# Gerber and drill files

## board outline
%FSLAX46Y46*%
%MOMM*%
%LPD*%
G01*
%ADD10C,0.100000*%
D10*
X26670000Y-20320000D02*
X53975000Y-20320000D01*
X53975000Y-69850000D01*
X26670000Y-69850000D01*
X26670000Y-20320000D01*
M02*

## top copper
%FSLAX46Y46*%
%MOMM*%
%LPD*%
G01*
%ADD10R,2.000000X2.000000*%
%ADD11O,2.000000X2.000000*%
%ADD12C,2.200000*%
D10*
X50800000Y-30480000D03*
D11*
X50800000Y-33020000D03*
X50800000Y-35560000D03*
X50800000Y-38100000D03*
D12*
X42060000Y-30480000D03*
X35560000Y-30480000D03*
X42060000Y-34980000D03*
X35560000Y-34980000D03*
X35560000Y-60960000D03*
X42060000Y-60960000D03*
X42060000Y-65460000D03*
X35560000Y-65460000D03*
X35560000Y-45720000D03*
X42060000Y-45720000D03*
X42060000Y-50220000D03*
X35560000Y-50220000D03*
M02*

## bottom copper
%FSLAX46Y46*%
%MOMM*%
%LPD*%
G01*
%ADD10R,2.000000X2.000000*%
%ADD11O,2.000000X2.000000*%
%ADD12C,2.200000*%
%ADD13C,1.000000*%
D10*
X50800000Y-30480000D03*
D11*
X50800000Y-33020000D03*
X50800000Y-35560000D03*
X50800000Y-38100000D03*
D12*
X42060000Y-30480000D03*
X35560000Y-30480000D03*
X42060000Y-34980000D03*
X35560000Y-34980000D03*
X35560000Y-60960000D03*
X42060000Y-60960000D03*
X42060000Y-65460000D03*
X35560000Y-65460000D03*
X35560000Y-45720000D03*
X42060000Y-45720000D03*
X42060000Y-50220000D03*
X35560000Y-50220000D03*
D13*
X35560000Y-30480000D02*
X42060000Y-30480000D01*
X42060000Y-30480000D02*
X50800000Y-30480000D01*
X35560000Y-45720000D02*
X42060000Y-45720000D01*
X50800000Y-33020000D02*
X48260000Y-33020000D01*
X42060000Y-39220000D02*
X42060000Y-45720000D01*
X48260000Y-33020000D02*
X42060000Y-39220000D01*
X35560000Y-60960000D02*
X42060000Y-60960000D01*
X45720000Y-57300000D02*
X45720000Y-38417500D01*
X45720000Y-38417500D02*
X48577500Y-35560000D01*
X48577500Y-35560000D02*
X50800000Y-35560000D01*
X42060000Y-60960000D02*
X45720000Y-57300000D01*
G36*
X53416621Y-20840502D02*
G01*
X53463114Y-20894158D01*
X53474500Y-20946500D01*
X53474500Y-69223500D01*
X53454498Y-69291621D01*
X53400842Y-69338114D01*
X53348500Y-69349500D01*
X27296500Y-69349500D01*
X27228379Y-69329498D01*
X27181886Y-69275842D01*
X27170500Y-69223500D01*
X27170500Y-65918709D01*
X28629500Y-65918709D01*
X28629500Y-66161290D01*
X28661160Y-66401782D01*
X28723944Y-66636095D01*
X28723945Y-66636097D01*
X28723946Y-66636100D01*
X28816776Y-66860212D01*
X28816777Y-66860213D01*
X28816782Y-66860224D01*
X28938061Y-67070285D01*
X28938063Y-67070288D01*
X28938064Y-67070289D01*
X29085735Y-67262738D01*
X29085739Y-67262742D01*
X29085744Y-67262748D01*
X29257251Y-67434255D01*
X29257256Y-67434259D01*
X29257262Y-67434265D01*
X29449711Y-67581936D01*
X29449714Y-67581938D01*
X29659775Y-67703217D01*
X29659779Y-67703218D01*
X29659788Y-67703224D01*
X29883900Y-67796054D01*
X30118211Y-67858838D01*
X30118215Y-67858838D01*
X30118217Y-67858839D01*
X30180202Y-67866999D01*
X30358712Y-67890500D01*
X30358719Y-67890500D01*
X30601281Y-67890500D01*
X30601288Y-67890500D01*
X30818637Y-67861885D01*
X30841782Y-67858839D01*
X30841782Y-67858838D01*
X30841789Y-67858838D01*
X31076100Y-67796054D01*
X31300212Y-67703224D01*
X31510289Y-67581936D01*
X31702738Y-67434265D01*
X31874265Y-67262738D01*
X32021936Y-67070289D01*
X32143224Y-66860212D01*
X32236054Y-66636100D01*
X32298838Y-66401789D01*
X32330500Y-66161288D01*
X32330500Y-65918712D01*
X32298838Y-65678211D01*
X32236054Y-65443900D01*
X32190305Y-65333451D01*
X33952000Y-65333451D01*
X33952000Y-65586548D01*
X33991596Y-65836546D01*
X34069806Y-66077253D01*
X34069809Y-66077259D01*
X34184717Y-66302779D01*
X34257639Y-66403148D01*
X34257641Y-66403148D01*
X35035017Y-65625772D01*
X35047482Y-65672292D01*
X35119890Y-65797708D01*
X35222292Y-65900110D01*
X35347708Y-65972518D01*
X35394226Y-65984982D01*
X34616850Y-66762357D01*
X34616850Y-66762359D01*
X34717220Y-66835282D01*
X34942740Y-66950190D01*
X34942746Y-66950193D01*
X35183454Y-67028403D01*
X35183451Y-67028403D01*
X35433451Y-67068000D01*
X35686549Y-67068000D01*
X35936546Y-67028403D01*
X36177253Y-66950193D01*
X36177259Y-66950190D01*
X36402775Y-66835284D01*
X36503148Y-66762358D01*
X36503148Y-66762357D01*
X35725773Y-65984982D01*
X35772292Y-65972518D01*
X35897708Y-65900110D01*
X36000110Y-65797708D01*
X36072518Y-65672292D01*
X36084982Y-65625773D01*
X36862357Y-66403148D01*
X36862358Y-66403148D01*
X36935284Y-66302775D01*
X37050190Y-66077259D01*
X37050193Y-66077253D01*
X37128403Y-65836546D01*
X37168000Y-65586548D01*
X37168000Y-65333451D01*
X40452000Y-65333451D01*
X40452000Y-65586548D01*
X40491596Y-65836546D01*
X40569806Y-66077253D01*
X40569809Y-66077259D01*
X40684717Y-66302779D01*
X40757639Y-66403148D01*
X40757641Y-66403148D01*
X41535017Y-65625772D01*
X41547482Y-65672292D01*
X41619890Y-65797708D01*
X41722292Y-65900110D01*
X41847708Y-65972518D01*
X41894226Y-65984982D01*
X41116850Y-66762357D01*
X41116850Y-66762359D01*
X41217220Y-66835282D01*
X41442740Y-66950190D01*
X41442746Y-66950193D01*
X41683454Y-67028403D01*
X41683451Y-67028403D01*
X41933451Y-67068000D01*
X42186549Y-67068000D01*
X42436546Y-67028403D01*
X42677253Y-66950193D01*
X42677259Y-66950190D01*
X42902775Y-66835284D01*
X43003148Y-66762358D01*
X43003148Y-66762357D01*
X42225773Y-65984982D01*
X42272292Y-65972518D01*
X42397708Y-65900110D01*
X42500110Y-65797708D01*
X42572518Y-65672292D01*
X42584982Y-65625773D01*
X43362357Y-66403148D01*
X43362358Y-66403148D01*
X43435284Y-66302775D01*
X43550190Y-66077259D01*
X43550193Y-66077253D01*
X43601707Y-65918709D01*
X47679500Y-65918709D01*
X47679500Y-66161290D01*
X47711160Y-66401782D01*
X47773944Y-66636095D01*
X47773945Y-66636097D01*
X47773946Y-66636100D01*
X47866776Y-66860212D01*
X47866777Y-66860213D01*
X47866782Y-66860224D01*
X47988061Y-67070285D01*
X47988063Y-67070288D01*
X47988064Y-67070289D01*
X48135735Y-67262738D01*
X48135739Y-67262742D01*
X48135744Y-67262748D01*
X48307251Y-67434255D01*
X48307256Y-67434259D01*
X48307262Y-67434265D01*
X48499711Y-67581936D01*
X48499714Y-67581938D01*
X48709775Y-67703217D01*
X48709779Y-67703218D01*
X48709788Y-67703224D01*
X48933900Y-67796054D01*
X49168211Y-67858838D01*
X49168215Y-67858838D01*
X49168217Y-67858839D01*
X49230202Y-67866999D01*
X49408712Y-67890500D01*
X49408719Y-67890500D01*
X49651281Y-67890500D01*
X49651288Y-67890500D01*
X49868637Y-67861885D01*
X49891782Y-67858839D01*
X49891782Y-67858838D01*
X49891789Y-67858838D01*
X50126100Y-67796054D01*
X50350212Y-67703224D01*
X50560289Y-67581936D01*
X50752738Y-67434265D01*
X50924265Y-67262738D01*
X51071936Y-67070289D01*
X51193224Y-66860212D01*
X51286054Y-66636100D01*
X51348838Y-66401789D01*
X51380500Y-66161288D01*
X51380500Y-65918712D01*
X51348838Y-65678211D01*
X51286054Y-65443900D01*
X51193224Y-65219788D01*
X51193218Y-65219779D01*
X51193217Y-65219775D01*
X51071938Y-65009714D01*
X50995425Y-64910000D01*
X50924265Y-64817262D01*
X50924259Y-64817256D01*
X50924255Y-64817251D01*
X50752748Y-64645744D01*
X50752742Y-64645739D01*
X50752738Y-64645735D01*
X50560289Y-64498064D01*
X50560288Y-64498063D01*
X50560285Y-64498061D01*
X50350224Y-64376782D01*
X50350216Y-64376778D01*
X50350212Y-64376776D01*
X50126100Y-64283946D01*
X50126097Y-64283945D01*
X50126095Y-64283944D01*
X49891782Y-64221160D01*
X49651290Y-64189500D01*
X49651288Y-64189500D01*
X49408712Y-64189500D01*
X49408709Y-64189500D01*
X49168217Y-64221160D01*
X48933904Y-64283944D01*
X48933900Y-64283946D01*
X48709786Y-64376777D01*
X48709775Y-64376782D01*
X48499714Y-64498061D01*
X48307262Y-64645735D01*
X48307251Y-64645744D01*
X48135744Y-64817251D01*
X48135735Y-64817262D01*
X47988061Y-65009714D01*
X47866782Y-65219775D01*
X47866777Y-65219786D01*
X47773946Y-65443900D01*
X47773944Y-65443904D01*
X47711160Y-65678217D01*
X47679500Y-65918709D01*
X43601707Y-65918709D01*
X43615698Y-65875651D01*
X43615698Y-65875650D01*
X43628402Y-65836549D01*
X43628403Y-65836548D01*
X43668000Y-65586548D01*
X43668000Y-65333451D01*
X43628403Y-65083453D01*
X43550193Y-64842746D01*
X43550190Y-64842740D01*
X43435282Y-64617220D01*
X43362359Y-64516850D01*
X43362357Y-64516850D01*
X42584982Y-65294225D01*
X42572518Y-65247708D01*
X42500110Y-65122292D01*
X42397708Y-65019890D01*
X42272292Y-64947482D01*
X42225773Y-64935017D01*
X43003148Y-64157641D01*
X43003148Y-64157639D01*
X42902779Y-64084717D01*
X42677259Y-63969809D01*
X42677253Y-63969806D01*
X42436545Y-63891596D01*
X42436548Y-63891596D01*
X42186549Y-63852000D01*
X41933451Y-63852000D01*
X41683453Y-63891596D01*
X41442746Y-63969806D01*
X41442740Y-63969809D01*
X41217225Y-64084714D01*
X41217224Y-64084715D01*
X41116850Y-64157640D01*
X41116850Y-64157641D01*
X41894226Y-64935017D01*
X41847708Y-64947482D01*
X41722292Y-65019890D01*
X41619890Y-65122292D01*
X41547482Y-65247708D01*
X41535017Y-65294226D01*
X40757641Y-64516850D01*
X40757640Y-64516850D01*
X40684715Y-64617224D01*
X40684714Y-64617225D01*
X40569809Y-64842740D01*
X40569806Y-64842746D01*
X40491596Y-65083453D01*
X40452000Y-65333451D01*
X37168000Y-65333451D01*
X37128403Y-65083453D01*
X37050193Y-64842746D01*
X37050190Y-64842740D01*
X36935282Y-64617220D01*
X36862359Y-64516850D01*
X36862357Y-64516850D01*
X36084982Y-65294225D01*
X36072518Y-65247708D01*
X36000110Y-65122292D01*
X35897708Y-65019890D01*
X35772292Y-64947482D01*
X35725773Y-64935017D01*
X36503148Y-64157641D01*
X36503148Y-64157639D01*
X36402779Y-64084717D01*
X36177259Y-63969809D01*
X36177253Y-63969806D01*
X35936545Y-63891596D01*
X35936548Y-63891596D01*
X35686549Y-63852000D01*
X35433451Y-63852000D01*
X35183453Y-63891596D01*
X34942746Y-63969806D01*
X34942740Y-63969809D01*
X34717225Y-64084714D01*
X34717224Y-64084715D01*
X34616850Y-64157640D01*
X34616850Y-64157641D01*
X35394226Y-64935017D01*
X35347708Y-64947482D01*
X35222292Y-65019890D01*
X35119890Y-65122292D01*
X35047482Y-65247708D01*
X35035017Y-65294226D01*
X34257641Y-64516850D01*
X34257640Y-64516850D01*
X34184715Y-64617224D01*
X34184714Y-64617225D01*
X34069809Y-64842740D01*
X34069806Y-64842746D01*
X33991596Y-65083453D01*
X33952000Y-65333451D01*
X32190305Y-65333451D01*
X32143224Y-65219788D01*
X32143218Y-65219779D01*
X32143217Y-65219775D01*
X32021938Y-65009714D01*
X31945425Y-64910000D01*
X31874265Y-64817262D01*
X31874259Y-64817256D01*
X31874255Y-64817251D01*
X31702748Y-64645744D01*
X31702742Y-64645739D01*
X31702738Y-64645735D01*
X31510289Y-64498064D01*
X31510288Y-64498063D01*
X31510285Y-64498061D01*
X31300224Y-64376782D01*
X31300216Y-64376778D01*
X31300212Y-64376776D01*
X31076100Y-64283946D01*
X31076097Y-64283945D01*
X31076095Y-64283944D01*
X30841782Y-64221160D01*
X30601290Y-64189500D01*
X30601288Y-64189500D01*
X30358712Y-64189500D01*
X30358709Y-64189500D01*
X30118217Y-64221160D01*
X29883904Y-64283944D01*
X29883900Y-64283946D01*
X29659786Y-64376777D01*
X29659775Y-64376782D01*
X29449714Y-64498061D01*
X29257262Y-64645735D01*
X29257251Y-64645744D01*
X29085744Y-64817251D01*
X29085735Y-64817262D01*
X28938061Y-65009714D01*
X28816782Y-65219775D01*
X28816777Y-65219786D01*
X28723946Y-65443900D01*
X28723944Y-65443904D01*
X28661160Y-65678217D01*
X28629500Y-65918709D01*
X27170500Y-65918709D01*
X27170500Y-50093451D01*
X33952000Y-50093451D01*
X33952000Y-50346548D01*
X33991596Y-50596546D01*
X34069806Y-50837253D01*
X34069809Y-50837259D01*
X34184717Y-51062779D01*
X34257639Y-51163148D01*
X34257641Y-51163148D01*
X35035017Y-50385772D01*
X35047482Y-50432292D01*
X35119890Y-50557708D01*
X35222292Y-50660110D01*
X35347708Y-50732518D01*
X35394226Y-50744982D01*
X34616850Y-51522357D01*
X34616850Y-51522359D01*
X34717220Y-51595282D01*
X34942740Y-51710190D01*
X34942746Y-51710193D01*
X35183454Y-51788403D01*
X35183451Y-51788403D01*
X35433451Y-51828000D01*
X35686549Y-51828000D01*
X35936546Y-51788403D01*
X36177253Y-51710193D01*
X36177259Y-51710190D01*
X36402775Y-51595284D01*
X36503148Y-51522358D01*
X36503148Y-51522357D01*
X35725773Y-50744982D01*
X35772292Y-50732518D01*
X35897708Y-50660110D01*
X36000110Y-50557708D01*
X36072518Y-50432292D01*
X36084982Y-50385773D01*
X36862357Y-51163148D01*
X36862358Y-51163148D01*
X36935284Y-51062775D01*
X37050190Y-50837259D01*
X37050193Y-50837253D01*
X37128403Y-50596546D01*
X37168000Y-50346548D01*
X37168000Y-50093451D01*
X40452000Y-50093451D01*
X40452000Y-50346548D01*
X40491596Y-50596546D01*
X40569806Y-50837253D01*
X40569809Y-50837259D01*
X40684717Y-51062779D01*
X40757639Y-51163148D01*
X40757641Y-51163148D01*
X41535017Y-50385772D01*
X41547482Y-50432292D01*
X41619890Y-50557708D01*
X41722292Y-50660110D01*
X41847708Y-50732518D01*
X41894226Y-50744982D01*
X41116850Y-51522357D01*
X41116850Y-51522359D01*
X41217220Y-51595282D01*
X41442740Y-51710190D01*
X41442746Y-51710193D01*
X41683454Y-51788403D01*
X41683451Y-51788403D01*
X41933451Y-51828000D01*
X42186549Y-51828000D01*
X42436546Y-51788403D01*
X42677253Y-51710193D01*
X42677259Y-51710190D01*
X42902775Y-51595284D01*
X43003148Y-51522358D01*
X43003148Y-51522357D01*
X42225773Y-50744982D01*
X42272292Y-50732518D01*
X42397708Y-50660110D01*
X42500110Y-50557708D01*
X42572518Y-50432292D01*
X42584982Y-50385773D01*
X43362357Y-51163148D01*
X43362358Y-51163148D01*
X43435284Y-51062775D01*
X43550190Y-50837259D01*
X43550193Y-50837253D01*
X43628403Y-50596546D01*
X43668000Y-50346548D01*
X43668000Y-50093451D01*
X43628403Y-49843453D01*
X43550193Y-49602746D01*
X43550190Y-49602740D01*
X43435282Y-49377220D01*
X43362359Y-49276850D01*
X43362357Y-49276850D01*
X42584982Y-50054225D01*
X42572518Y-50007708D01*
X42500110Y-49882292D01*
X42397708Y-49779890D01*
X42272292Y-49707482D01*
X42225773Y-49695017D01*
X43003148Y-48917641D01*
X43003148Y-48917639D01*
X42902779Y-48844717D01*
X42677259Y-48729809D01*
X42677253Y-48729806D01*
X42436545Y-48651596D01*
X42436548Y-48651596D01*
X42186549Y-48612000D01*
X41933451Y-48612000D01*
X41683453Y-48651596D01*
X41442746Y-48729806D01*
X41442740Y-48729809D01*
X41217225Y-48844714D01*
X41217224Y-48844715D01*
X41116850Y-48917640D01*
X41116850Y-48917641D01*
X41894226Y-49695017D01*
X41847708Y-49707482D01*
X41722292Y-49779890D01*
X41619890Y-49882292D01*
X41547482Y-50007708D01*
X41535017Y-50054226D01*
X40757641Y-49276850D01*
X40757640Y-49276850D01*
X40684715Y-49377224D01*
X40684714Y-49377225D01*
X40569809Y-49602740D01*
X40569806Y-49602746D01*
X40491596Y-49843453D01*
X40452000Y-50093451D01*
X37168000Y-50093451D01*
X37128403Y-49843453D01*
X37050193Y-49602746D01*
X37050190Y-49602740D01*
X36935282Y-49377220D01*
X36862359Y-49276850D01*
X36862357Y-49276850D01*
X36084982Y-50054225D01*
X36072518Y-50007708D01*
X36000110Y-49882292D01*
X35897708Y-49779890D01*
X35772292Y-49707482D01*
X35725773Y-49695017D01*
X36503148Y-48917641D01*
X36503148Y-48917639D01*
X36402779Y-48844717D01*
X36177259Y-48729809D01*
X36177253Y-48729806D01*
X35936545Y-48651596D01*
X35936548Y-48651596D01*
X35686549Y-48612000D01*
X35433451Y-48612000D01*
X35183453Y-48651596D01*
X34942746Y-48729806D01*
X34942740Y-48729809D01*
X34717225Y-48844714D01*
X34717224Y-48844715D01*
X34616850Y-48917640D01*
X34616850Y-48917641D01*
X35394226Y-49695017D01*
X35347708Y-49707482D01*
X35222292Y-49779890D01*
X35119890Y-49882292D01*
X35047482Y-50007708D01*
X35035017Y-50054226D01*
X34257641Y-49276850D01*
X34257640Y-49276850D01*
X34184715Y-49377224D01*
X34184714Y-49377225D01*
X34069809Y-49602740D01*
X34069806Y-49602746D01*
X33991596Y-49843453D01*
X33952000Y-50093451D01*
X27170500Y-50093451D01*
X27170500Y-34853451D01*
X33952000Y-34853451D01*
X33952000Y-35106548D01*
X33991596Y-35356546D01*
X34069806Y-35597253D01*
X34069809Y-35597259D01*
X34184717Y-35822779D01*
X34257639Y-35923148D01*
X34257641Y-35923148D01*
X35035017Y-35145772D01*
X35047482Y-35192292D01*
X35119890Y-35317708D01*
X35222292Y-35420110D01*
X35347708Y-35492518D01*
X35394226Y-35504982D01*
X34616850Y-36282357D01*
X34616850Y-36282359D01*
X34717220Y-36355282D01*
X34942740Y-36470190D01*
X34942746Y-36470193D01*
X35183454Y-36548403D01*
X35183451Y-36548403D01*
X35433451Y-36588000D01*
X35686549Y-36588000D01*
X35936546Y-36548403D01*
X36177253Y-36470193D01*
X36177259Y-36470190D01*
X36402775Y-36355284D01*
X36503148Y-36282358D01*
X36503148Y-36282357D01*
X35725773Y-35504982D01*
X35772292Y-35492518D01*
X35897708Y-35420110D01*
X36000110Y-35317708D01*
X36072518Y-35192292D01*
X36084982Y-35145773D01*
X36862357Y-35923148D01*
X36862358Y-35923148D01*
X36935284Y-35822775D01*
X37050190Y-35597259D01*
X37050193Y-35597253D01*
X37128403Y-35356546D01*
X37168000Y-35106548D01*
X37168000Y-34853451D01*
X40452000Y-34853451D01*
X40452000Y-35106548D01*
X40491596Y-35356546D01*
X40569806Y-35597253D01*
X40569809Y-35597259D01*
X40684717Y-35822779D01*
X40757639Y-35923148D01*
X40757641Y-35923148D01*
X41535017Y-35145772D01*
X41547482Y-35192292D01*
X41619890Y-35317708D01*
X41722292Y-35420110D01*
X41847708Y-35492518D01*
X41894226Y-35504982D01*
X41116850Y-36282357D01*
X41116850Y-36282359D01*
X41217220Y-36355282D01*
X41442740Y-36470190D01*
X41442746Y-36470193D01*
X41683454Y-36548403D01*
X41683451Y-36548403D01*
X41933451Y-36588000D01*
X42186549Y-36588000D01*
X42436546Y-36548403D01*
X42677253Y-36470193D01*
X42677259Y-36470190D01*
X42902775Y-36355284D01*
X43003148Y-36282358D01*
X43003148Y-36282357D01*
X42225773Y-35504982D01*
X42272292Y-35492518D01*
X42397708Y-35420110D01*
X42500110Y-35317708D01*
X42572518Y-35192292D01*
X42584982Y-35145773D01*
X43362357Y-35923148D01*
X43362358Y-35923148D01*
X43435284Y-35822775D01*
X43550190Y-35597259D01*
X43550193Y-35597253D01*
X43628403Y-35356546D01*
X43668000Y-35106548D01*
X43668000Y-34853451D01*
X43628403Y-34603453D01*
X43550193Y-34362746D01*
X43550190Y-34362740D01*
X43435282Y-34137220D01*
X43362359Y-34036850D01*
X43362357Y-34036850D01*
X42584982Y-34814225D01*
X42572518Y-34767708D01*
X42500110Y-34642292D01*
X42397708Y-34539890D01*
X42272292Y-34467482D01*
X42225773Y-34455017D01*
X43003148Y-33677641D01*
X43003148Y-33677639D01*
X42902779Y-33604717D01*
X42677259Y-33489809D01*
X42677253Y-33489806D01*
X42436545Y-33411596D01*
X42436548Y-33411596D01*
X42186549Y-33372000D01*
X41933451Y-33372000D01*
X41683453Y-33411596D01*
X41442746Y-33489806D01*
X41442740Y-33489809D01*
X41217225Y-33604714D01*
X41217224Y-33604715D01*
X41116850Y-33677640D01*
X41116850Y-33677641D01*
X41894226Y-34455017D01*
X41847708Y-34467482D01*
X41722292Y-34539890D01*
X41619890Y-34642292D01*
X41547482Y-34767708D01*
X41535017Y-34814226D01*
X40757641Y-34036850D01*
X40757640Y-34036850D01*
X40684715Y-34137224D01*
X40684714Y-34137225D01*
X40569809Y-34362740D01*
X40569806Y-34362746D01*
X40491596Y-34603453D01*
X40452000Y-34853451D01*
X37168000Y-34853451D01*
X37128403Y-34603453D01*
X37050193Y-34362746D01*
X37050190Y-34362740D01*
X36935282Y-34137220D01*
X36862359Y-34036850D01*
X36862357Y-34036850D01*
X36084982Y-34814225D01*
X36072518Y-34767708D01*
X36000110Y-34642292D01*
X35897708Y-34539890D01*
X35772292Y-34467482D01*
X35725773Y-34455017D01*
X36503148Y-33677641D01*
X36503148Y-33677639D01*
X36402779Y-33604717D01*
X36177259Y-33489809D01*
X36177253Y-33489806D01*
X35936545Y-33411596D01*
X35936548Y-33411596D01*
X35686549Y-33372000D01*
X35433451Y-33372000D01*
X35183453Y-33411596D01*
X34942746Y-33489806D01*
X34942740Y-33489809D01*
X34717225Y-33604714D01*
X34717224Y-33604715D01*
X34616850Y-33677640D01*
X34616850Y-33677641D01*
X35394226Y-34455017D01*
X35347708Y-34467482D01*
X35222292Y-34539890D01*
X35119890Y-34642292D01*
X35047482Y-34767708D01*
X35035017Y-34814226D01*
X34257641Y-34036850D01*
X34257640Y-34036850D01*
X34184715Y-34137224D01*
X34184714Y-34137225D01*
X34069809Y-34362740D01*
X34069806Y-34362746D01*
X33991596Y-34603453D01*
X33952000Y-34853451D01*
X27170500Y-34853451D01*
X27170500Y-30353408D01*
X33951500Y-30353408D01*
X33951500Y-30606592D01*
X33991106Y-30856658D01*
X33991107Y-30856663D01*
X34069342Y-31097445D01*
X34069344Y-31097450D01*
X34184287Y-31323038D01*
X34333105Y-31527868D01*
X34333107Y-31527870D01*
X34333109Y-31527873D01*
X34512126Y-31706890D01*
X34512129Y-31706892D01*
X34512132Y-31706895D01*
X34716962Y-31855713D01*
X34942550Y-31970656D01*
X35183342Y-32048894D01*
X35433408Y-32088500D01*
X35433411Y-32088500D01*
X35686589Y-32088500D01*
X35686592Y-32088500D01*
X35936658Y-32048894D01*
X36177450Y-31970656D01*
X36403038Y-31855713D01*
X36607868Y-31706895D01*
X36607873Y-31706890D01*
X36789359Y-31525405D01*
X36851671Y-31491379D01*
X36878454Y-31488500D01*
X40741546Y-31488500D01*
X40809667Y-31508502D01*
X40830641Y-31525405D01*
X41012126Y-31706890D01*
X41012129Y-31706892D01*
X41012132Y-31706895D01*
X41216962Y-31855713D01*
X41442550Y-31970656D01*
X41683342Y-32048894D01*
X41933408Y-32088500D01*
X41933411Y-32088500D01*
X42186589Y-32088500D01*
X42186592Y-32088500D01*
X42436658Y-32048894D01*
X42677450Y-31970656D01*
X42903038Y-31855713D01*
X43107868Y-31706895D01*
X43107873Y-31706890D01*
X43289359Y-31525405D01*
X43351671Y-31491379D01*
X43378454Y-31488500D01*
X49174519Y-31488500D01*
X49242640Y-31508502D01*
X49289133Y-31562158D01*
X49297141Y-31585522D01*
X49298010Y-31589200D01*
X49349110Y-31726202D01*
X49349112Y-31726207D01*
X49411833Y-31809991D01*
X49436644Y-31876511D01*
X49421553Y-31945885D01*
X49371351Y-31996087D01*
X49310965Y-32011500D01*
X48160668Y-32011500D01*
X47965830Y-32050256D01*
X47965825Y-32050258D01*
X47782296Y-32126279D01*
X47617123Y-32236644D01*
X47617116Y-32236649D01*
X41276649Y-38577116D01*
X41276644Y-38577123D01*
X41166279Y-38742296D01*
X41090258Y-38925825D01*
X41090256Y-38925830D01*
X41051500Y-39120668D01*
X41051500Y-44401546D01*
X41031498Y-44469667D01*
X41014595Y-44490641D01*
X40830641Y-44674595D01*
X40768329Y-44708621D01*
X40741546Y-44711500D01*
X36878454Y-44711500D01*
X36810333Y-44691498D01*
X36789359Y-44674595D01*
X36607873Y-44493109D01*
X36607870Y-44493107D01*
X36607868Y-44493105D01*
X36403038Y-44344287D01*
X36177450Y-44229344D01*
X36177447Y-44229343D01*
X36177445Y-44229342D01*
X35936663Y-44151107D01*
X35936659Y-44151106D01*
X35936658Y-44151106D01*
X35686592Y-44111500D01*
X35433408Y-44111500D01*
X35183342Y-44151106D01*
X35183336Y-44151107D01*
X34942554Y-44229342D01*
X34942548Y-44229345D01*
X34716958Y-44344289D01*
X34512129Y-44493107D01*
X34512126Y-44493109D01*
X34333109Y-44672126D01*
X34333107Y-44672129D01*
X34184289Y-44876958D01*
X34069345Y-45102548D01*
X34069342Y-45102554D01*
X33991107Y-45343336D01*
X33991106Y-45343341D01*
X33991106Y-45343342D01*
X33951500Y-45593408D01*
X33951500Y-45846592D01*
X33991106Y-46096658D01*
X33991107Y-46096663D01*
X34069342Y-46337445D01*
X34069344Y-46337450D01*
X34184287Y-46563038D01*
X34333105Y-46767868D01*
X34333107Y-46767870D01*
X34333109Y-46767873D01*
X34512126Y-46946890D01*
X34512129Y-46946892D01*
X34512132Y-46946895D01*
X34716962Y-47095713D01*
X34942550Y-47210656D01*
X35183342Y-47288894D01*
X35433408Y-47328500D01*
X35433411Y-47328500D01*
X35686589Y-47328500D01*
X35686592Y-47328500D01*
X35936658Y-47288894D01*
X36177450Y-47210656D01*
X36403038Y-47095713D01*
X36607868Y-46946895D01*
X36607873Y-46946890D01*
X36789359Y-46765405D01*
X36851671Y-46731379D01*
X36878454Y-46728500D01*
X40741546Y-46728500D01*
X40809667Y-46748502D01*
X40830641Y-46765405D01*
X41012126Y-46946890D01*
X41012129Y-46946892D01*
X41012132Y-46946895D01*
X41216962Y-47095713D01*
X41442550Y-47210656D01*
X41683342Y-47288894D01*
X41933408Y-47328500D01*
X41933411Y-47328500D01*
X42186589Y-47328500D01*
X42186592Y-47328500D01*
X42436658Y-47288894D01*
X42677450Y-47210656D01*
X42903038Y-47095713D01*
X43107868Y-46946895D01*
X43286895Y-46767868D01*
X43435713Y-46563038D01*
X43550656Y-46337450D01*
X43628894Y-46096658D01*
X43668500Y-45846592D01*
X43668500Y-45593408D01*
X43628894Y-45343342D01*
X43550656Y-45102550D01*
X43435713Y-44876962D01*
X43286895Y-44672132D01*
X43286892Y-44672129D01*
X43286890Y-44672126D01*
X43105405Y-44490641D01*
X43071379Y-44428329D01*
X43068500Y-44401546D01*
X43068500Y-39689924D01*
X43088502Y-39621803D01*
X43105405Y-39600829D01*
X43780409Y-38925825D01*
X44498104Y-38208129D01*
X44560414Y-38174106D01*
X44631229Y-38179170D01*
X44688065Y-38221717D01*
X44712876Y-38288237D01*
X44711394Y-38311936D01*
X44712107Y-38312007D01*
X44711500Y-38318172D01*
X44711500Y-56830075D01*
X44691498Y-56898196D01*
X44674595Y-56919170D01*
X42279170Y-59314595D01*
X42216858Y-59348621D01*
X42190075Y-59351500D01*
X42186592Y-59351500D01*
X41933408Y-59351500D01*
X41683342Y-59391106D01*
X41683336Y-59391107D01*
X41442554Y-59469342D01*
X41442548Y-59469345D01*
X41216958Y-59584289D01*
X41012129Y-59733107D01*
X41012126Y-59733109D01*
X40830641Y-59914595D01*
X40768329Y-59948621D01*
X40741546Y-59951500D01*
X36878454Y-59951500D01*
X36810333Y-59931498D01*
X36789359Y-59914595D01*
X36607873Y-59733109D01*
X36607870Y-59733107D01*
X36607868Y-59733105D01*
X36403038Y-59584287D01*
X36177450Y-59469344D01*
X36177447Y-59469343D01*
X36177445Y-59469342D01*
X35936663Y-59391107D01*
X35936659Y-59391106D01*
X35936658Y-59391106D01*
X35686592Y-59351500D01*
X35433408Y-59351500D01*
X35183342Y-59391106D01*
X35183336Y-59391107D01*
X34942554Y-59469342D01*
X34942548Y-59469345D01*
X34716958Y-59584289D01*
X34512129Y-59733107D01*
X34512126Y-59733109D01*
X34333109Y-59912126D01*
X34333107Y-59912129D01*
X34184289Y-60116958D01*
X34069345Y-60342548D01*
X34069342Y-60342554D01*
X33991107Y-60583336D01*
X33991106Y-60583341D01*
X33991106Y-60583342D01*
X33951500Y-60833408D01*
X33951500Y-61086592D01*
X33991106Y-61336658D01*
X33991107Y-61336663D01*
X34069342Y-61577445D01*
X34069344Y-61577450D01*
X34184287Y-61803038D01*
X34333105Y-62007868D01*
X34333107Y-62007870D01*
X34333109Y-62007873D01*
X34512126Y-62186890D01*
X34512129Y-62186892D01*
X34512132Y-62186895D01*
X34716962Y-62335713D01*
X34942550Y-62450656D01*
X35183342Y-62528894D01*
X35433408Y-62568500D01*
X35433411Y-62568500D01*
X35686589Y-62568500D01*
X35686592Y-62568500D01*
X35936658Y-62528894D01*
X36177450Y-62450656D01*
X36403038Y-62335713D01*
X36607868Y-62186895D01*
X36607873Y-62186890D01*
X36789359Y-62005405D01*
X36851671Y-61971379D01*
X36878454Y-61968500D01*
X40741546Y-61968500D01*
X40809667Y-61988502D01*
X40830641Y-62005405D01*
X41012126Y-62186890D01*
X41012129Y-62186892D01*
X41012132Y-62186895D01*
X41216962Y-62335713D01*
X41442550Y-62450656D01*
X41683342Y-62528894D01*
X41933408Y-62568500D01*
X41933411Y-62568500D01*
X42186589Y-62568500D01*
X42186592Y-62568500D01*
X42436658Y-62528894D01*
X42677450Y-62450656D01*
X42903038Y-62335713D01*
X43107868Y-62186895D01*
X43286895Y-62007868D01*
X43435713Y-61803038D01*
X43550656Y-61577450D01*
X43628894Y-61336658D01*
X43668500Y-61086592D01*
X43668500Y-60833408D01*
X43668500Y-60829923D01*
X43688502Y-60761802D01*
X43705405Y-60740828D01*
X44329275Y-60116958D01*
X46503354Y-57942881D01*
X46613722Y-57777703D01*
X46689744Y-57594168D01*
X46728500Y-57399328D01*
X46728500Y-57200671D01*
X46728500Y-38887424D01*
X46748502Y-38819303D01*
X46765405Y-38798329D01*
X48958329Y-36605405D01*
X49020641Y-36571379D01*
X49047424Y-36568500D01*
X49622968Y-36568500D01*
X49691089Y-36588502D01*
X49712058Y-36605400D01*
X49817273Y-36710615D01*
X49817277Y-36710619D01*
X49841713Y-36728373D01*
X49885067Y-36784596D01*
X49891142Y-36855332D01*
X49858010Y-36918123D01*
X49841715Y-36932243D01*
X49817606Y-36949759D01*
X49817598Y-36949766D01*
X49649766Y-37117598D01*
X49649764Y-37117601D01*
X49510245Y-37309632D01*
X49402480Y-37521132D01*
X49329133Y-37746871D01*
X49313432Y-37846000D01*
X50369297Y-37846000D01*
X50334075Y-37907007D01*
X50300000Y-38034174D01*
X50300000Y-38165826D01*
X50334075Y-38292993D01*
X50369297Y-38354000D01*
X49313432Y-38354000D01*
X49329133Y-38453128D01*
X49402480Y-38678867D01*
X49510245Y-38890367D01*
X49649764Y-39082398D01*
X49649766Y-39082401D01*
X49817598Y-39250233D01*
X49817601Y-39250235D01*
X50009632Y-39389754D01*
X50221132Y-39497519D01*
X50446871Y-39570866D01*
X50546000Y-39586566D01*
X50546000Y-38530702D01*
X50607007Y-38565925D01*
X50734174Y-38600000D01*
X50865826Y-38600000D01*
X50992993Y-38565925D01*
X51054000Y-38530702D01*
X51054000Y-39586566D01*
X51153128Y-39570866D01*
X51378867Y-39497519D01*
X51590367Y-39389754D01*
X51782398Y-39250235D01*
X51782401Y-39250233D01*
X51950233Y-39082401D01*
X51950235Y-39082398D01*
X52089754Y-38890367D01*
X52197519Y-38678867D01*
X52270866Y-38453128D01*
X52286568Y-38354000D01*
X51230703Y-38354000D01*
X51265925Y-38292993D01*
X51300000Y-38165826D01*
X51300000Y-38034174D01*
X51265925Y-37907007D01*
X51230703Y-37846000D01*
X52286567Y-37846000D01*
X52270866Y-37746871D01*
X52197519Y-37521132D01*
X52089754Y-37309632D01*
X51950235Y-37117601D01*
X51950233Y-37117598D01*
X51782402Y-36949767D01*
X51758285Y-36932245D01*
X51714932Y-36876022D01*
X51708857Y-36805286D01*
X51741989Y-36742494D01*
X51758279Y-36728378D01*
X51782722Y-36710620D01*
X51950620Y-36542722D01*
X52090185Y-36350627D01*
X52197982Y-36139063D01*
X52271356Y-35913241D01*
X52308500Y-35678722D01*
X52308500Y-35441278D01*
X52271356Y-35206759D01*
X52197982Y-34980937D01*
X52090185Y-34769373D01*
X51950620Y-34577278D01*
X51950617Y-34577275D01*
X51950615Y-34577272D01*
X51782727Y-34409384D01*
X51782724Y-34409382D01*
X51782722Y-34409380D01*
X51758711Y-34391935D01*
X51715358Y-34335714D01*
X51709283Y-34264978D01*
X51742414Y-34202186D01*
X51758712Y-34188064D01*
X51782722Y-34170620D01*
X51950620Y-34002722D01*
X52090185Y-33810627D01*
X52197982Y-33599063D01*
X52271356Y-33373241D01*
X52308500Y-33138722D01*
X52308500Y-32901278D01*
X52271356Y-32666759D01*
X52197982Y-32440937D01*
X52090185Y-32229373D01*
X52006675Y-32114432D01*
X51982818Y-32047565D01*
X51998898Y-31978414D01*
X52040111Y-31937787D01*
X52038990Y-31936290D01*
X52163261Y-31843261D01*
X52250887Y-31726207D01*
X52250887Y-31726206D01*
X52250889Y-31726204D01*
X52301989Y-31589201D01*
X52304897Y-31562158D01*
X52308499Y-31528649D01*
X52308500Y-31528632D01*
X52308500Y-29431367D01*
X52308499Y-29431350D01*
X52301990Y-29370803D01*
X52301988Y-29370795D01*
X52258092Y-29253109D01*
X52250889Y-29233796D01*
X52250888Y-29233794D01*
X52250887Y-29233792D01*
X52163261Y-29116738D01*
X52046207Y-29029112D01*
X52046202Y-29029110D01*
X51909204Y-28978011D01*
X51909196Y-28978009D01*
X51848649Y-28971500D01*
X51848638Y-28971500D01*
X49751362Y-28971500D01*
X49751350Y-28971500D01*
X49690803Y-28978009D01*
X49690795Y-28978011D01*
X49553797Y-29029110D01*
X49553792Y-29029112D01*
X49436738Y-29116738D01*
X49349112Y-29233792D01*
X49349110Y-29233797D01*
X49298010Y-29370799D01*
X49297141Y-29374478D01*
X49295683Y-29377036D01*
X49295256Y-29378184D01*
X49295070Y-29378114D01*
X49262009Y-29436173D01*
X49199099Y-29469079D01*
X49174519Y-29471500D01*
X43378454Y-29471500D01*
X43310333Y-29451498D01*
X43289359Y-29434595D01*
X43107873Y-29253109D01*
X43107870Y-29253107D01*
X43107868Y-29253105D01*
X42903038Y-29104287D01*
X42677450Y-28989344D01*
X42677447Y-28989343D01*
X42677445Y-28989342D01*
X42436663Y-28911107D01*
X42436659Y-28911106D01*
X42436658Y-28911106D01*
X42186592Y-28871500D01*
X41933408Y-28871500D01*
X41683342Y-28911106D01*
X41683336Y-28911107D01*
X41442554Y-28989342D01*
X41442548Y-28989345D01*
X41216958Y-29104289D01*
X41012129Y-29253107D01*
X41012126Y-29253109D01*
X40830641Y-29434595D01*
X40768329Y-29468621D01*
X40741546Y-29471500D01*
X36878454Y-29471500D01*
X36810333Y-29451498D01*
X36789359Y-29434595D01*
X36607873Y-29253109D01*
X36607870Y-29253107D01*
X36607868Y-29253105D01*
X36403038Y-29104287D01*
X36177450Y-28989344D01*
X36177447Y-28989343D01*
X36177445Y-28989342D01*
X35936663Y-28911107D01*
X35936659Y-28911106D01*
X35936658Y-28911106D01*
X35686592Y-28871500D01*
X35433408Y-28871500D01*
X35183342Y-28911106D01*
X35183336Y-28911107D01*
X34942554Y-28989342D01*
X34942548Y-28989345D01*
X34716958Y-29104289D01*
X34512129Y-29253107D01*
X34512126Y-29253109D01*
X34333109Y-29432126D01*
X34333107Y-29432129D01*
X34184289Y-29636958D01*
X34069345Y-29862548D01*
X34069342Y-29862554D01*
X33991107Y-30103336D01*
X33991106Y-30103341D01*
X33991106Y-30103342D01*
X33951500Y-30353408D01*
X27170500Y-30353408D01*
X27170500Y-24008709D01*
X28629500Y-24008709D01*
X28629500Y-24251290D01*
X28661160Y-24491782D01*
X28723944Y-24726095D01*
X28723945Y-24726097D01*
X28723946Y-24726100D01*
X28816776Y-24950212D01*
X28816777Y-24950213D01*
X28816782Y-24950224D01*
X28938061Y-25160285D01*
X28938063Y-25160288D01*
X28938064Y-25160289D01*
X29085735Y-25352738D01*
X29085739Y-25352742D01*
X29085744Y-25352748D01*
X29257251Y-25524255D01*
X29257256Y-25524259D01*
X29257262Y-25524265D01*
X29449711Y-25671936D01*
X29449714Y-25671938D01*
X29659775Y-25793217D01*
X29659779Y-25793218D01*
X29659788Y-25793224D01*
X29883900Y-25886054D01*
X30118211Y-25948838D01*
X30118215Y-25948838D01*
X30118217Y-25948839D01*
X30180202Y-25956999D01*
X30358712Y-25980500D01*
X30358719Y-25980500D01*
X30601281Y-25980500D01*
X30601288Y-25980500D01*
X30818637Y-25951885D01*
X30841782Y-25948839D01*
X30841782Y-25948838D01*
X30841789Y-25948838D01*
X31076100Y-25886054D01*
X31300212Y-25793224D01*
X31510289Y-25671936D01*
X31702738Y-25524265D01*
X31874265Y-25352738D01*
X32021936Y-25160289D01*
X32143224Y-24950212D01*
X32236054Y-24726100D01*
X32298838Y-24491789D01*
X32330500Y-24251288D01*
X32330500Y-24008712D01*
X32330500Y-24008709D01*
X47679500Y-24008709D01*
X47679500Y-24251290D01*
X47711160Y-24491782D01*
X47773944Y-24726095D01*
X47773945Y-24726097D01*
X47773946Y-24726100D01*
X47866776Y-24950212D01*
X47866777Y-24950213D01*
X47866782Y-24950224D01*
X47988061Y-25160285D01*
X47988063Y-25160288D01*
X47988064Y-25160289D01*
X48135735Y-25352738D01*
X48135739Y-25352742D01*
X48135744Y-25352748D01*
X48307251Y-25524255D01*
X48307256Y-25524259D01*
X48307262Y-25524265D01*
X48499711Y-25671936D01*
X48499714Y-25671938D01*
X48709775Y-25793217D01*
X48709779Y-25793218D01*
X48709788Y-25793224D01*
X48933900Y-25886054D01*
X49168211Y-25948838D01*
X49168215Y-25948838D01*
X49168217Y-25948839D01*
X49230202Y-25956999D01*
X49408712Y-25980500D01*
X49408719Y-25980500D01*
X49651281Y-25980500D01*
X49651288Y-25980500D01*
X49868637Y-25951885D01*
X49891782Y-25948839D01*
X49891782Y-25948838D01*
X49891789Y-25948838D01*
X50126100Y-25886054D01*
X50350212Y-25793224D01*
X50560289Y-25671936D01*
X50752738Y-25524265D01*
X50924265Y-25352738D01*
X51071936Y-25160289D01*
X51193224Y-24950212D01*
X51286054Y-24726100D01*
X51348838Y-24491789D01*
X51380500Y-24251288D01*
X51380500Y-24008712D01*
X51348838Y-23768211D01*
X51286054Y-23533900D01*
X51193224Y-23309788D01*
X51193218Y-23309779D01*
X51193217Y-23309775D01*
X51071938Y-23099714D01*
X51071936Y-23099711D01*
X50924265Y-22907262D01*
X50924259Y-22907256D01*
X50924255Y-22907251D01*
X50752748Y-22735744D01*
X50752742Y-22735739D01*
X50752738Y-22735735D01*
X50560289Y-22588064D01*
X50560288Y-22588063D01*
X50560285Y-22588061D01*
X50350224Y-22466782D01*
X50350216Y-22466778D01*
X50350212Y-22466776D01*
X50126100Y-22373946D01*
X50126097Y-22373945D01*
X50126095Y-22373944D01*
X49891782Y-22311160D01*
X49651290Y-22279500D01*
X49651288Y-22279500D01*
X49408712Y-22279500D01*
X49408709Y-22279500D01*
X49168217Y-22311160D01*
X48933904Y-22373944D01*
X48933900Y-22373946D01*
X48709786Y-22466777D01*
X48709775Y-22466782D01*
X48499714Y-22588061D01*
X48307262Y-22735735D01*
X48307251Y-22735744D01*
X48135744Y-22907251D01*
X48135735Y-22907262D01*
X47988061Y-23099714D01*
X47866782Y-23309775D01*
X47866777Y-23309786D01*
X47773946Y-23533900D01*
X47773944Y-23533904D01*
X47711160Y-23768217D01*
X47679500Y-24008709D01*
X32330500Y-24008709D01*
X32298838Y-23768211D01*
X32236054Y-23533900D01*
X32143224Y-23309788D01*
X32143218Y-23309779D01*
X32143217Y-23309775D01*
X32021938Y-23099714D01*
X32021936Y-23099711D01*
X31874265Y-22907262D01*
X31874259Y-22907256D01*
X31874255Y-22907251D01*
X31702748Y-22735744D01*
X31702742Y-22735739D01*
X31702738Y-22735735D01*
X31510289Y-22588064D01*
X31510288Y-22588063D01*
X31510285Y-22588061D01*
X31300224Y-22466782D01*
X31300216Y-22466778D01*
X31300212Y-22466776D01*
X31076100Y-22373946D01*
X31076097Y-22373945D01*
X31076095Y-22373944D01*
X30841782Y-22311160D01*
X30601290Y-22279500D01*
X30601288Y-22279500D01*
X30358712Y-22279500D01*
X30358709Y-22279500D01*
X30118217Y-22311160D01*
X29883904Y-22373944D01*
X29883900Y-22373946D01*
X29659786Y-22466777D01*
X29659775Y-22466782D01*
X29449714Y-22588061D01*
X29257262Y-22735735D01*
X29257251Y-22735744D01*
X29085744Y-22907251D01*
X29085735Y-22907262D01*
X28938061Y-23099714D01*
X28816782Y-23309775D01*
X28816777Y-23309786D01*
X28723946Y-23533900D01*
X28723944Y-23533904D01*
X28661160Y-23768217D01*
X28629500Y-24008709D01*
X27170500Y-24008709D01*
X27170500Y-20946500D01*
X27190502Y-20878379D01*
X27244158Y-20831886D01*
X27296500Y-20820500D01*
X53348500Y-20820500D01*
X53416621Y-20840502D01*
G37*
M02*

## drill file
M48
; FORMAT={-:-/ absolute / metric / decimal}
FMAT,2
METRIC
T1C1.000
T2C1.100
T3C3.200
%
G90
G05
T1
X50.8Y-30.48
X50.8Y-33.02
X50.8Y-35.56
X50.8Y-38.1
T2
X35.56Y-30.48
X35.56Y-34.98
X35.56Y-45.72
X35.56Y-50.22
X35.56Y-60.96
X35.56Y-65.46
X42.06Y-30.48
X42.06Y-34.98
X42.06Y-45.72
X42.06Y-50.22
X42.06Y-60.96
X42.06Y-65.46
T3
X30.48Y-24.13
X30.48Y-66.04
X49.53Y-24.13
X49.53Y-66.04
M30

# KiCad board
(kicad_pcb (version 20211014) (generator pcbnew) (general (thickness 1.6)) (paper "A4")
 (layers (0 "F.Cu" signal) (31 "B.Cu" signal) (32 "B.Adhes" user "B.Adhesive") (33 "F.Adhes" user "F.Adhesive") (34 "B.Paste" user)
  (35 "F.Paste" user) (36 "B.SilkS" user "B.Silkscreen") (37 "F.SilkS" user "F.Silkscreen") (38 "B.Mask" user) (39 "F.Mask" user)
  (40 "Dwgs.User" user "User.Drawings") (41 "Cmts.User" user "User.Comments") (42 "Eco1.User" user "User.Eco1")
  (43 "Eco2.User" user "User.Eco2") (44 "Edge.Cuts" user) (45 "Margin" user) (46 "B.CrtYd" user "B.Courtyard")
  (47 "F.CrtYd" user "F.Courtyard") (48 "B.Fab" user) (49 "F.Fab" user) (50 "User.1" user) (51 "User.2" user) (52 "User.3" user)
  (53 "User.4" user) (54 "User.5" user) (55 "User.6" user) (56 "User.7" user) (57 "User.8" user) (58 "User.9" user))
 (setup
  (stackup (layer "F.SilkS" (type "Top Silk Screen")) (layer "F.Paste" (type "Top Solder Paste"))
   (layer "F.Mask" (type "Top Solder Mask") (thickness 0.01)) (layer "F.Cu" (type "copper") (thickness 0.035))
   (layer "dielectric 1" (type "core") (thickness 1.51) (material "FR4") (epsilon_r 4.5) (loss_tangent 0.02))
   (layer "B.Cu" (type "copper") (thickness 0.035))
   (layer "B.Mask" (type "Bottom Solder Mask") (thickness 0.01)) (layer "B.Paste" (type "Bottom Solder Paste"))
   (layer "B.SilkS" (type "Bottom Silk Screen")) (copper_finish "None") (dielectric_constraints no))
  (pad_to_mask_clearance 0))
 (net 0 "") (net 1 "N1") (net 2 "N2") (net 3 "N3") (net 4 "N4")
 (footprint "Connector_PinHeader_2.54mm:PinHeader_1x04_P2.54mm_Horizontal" (layer "F.Cu") (at 50.8 30.48)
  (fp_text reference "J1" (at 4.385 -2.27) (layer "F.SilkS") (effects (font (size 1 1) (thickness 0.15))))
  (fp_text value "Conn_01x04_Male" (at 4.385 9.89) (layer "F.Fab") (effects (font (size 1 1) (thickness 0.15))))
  (pad "1" thru_hole rect (at 0 0) (size 2 2) (drill 1) (layers *.Cu *.Mask) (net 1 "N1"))
  (pad "2" thru_hole oval (at 0 2.54) (size 2 2) (drill 1) (layers *.Cu *.Mask) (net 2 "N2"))
  (pad "3" thru_hole oval (at 0 5.08) (size 2 2) (drill 1) (layers *.Cu *.Mask) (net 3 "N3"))
  (pad "4" thru_hole oval (at 0 7.62) (size 2 2) (drill 1) (layers *.Cu *.Mask) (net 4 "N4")))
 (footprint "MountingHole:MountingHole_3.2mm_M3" (layer "F.Cu") (at 30.48 66.04)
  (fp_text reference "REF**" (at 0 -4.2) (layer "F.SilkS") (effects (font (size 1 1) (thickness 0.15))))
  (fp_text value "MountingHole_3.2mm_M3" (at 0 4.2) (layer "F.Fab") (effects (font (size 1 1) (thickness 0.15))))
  (pad "" np_thru_hole circle (at 0 0) (size 3.2 3.2) (drill 3.2) (layers *.Cu *.Mask)))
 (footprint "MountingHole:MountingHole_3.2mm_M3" (layer "F.Cu") (at 49.53 66.04)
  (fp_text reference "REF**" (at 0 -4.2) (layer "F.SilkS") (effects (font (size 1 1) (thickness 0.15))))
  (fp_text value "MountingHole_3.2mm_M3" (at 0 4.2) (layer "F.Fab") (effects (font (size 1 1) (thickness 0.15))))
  (pad "" np_thru_hole circle (at 0 0) (size 3.2 3.2) (drill 3.2) (layers *.Cu *.Mask)))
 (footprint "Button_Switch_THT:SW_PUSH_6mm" (layer "F.Cu") (at 35.56 30.48)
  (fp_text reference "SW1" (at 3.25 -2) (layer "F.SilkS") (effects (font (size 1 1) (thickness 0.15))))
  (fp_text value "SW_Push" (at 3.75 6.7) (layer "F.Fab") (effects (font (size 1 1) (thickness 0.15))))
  (pad "1" thru_hole circle (at 6.5 0 90) (size 2.2 2.2) (drill 1.1) (layers *.Cu *.Mask) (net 1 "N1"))
  (pad "1" thru_hole circle (at 0 0 90) (size 2.2 2.2) (drill 1.1) (layers *.Cu *.Mask) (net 1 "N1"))
  (pad "2" thru_hole circle (at 6.5 4.5 90) (size 2.2 2.2) (drill 1.1) (layers *.Cu *.Mask) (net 4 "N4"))
  (pad "2" thru_hole circle (at 0 4.5 90) (size 2.2 2.2) (drill 1.1) (layers *.Cu *.Mask) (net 4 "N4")))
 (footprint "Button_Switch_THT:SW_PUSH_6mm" (layer "F.Cu") (at 35.56 60.96)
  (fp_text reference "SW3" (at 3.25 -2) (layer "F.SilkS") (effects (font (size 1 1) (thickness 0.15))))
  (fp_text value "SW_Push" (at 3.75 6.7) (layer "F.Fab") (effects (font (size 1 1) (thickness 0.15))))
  (pad "1" thru_hole circle (at 0 0 90) (size 2.2 2.2) (drill 1.1) (layers *.Cu *.Mask) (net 3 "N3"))
  (pad "1" thru_hole circle (at 6.5 0 90) (size 2.2 2.2) (drill 1.1) (layers *.Cu *.Mask) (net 3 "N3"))
  (pad "2" thru_hole circle (at 6.5 4.5 90) (size 2.2 2.2) (drill 1.1) (layers *.Cu *.Mask) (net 4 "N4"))
  (pad "2" thru_hole circle (at 0 4.5 90) (size 2.2 2.2) (drill 1.1) (layers *.Cu *.Mask) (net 4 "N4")))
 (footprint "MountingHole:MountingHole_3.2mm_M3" (layer "F.Cu") (at 30.48 24.13)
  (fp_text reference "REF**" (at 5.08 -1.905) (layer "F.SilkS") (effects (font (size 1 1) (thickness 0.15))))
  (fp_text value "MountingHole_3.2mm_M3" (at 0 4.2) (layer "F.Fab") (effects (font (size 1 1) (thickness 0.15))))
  (pad "" np_thru_hole circle (at 0 0) (size 3.2 3.2) (drill 3.2) (layers *.Cu *.Mask)))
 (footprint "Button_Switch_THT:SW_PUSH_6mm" (layer "F.Cu") (at 35.56 45.72)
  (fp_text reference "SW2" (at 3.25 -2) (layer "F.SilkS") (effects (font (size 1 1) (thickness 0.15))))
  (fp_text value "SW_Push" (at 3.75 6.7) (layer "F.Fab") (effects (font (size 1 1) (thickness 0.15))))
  (pad "1" thru_hole circle (at 0 0 90) (size 2.2 2.2) (drill 1.1) (layers *.Cu *.Mask) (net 2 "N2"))
  (pad "1" thru_hole circle (at 6.5 0 90) (size 2.2 2.2) (drill 1.1) (layers *.Cu *.Mask "Dwgs.User") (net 2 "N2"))
  (pad "2" thru_hole circle (at 6.5 4.5 90) (size 2.2 2.2) (drill 1.1) (layers *.Cu *.Mask) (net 4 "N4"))
  (pad "2" thru_hole circle (at 0 4.5 90) (size 2.2 2.2) (drill 1.1) (layers *.Cu *.Mask) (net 4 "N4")))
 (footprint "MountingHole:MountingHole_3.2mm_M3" (layer "F.Cu") (at 49.53 24.13)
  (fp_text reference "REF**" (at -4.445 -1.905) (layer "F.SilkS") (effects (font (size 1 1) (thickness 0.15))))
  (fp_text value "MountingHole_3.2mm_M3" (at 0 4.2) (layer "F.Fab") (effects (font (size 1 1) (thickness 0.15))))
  (pad "" np_thru_hole circle (at 0 0) (size 3.2 3.2) (drill 3.2) (layers *.Cu *.Mask)))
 (gr_rect (start 26.67 20.32) (end 53.975 69.85) (layer "Edge.Cuts") (width 0.1) (fill none))
 (segment (start 35.56 30.48) (end 42.06 30.48) (width 1) (layer "B.Cu") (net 1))
 (segment (start 42.06 30.48) (end 50.8 30.48) (width 1) (layer "B.Cu") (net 1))
 (segment (start 35.56 45.72) (end 42.06 45.72) (width 1) (layer "B.Cu") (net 2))
 (segment (start 50.8 33.02) (end 48.26 33.02) (width 1) (layer "B.Cu") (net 2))
 (segment (start 42.06 39.22) (end 42.06 45.72) (width 1) (layer "B.Cu") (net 2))
 (segment (start 48.26 33.02) (end 42.06 39.22) (width 1) (layer "B.Cu") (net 2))
 (segment (start 35.56 60.96) (end 42.06 60.96) (width 1) (layer "B.Cu") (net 3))
 (segment (start 45.72 57.3) (end 45.72 38.4175) (width 1) (layer "B.Cu") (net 3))
 (segment (start 45.72 38.4175) (end 48.5775 35.56) (width 1) (layer "B.Cu") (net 3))
 (segment (start 48.5775 35.56) (end 50.8 35.56) (width 1) (layer "B.Cu") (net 3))
 (segment (start 42.06 60.96) (end 45.72 57.3) (width 1) (layer "B.Cu") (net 3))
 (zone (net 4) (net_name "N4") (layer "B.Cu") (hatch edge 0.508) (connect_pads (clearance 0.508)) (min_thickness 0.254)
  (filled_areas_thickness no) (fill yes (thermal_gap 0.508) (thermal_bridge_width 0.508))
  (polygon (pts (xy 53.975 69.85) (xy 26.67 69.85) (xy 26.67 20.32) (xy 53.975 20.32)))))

